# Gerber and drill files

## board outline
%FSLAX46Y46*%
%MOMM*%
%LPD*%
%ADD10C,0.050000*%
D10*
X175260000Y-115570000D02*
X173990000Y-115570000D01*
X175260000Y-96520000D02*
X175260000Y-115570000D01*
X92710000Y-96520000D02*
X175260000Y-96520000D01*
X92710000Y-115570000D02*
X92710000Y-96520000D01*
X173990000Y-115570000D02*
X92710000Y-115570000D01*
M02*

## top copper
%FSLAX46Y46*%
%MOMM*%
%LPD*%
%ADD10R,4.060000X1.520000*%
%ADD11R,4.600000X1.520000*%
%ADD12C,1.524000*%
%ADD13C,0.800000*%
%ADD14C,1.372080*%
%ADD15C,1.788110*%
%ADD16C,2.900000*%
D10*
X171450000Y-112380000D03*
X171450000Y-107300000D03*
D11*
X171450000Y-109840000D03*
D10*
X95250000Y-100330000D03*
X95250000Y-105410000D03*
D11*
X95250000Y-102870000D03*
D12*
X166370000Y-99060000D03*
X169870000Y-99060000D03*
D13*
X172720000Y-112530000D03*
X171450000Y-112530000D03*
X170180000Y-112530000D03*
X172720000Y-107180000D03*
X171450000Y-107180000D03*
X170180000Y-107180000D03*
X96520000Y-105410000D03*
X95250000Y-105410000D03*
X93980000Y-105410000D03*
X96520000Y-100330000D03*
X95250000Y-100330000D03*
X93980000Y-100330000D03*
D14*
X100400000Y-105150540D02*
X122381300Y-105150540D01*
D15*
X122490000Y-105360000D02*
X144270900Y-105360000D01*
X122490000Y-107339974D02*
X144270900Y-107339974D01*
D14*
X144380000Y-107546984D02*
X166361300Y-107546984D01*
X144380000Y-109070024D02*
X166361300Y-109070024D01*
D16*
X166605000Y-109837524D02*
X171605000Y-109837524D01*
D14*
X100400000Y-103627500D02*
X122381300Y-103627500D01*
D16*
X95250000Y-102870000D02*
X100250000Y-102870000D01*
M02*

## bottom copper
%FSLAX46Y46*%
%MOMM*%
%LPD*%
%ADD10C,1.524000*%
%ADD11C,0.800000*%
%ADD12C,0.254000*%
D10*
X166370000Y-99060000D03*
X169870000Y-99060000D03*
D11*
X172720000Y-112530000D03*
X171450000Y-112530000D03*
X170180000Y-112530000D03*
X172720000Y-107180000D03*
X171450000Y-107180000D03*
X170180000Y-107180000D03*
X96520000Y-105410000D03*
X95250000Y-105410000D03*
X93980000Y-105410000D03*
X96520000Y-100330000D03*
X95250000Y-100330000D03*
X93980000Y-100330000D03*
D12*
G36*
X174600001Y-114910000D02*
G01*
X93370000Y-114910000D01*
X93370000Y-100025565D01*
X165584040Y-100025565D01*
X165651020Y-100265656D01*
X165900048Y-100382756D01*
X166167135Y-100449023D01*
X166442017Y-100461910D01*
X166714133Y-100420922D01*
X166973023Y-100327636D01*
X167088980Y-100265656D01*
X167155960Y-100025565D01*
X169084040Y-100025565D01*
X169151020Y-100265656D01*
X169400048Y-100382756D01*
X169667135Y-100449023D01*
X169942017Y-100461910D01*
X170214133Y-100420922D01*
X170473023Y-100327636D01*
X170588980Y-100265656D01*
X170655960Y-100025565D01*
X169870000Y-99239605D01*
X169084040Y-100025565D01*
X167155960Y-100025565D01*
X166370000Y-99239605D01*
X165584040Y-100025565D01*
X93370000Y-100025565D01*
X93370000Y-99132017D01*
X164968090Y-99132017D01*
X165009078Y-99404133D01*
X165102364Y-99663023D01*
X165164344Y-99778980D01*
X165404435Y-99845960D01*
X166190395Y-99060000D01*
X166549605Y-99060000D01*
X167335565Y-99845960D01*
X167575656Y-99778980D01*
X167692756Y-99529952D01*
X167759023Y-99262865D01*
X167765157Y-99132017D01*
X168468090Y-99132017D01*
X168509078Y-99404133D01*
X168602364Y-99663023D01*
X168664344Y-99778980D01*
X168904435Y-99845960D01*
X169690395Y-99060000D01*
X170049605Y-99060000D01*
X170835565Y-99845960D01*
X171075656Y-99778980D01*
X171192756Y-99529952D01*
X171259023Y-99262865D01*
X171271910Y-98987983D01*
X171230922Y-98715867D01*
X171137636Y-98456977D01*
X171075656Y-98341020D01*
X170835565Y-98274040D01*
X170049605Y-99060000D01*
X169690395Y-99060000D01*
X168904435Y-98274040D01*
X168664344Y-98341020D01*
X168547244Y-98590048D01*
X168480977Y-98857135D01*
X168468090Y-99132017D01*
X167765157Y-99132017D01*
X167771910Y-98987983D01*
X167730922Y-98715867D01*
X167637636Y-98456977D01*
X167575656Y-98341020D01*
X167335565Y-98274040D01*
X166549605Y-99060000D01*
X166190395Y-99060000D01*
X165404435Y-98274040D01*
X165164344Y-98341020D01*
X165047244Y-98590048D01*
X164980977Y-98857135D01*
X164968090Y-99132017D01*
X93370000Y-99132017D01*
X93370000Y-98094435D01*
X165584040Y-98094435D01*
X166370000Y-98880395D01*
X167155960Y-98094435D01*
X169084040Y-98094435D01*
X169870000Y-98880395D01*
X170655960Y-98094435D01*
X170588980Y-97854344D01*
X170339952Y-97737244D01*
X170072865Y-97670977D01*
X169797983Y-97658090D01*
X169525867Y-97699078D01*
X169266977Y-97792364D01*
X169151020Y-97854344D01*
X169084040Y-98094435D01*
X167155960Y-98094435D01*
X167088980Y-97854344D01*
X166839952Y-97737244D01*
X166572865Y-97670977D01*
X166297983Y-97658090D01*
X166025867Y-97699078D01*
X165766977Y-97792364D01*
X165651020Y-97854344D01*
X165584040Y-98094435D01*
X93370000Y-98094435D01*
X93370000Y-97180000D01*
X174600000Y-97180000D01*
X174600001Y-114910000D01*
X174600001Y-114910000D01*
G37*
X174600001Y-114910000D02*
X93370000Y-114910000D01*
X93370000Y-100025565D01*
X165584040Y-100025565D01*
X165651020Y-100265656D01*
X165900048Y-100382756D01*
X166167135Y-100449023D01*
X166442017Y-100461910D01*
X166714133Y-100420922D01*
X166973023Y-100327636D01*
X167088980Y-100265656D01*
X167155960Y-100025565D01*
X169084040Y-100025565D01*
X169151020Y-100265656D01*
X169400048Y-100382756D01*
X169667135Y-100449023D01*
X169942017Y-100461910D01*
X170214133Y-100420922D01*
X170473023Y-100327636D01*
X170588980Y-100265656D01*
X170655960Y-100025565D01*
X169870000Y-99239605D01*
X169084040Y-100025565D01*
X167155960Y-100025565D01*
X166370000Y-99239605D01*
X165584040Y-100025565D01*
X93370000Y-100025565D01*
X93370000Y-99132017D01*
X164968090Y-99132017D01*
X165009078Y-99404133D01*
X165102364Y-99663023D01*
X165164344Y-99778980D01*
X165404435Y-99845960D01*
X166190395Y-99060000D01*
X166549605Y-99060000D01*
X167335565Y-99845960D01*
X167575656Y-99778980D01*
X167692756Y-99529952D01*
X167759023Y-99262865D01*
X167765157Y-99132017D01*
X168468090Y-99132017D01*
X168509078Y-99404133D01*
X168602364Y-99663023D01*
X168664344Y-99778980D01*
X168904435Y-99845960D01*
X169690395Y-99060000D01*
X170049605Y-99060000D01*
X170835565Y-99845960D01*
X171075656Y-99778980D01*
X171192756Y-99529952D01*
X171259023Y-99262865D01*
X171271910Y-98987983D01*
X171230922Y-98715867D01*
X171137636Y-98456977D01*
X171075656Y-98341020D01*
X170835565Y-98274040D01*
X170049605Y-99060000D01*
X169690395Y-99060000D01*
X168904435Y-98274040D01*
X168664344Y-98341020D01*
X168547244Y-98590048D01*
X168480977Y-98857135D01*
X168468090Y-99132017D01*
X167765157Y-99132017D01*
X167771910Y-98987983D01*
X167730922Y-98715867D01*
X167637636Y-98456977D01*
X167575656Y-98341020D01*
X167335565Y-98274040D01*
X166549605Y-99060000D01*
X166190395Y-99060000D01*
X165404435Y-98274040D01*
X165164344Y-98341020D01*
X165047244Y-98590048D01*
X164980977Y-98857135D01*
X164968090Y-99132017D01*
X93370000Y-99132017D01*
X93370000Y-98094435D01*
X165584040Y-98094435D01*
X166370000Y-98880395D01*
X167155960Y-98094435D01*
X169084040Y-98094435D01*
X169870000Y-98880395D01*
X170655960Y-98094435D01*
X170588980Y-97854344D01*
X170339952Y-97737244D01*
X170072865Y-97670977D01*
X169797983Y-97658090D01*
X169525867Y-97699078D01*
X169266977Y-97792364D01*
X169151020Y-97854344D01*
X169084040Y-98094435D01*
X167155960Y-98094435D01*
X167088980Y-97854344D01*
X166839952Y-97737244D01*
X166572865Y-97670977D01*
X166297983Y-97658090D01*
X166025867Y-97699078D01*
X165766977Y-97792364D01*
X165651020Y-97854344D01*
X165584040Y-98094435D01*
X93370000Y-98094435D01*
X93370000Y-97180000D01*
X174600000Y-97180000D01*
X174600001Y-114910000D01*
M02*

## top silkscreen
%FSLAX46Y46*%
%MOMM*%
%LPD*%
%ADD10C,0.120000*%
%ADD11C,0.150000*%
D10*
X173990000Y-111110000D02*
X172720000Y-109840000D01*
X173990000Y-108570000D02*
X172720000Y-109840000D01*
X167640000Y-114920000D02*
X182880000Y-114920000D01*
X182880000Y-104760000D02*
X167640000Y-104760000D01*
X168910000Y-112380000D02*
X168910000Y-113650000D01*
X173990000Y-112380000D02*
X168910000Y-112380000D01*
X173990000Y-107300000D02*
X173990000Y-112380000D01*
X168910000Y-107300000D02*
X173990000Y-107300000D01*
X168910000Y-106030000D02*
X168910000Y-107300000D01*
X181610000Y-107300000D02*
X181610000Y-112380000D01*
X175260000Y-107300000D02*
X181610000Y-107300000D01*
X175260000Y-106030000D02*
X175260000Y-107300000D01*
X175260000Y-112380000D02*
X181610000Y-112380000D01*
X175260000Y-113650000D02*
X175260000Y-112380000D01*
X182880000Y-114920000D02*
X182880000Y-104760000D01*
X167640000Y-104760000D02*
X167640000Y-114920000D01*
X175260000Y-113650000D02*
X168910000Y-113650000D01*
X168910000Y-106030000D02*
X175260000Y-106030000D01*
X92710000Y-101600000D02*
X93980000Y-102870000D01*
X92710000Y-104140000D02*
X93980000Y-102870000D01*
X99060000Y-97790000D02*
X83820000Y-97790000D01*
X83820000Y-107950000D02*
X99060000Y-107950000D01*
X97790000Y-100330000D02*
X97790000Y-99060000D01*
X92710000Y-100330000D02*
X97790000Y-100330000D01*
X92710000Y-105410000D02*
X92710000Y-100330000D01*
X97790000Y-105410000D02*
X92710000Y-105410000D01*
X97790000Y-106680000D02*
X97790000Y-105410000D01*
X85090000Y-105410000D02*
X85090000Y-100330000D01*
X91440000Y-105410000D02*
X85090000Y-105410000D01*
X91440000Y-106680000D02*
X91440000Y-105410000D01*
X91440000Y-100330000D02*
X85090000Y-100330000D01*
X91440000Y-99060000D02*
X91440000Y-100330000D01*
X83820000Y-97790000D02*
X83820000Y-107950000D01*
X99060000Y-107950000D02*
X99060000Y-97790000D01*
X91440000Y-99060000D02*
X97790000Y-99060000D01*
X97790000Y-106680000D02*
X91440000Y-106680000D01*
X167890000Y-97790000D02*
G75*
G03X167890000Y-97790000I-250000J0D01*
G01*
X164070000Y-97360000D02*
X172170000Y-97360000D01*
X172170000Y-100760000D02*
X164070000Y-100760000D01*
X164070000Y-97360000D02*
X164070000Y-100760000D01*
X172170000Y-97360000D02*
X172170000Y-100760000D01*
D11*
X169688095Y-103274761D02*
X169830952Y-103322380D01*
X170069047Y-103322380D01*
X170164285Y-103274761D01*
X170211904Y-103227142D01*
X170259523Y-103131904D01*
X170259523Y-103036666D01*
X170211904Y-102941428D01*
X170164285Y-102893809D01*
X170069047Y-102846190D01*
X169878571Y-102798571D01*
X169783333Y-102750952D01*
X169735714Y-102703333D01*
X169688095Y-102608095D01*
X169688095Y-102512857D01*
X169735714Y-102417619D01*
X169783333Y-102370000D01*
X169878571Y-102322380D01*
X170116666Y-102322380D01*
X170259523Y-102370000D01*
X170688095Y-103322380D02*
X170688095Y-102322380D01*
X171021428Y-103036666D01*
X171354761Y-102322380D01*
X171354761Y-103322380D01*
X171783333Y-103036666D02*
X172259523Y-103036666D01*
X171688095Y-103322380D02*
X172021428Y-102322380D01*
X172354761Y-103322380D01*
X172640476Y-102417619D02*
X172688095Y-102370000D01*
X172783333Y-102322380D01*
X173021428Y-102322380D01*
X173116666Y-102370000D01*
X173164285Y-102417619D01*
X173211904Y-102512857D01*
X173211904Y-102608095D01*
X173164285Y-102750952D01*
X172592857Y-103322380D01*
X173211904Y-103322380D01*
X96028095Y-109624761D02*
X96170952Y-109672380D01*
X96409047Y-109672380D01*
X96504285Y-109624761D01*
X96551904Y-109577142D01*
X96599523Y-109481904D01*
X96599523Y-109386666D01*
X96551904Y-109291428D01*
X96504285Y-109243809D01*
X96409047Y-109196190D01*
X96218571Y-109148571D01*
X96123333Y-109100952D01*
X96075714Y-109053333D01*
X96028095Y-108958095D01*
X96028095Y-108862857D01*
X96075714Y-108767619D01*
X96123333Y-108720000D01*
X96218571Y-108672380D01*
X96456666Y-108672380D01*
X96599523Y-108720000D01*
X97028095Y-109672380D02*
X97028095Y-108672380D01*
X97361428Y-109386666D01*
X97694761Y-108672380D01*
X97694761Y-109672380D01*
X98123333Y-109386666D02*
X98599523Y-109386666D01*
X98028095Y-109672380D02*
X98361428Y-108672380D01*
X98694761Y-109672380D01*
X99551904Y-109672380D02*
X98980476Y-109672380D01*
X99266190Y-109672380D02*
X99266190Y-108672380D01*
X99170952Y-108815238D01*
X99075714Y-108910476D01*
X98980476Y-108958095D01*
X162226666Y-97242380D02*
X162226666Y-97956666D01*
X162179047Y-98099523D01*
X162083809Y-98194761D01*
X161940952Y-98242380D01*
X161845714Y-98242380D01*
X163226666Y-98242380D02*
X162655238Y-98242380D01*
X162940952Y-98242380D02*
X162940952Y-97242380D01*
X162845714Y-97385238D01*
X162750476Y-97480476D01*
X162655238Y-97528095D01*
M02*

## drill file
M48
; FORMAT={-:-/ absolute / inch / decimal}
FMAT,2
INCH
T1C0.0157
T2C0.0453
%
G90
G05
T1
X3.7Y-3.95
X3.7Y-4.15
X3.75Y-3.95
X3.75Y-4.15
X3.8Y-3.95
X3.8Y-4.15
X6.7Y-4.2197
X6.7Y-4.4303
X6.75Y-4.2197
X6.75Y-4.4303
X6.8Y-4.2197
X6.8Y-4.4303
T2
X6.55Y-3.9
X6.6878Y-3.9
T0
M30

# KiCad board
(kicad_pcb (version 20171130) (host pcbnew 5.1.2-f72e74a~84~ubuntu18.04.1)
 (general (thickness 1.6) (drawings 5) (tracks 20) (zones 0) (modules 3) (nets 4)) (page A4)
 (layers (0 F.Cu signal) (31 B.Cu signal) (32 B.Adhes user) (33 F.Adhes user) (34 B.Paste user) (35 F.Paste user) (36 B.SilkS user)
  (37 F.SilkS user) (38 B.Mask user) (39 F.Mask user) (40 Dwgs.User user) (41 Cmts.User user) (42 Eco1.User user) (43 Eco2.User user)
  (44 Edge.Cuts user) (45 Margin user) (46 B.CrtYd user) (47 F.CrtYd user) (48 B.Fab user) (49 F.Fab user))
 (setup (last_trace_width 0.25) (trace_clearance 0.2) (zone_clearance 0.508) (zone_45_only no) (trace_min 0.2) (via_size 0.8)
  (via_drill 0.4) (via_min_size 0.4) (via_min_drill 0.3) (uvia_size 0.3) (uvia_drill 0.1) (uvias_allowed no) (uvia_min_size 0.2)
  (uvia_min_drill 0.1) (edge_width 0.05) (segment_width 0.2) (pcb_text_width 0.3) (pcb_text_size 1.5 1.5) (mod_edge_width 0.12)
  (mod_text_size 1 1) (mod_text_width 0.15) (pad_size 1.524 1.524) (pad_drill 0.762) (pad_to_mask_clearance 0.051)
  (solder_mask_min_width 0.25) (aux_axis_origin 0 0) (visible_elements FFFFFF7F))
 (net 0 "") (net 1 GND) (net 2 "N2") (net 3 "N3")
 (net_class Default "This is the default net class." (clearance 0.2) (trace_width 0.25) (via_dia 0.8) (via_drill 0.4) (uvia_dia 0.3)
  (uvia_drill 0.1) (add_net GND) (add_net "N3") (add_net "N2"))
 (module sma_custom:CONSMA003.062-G (layer F.Cu) (at 175.26 112.38)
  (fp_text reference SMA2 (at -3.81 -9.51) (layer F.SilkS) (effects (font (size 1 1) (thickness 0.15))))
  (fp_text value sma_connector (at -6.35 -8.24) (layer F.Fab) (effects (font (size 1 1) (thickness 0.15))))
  (fp_line (start -1.27 -1.27) (end -2.54 -2.54) (layer F.SilkS) (width 0.12))
  (fp_line (start -1.27 -3.81) (end -2.54 -2.54) (layer F.SilkS) (width 0.12))
  (fp_line (start -7.62 2.54) (end 7.62 2.54) (layer F.SilkS) (width 0.12))
  (fp_line (start 7.62 -7.62) (end -7.62 -7.62) (layer F.SilkS) (width 0.12))
  (fp_line (start -6.35 0) (end -6.35 1.27) (layer F.SilkS) (width 0.12))
  (fp_line (start -1.27 0) (end -6.35 0) (layer F.SilkS) (width 0.12))
  (fp_line (start -1.27 -5.08) (end -1.27 0) (layer F.SilkS) (width 0.12))
  (fp_line (start -6.35 -5.08) (end -1.27 -5.08) (layer F.SilkS) (width 0.12))
  (fp_line (start -6.35 -6.35) (end -6.35 -5.08) (layer F.SilkS) (width 0.12))
  (fp_line (start 6.35 -5.08) (end 6.35 0) (layer F.SilkS) (width 0.12))
  (fp_line (start 0 -5.08) (end 6.35 -5.08) (layer F.SilkS) (width 0.12))
  (fp_line (start 0 -6.35) (end 0 -5.08) (layer F.SilkS) (width 0.12))
  (fp_line (start 0 0) (end 6.35 0) (layer F.SilkS) (width 0.12))
  (fp_line (start 0 1.27) (end 0 0) (layer F.SilkS) (width 0.12))
  (fp_line (start 7.62 2.54) (end 7.62 -7.62) (layer F.SilkS) (width 0.12))
  (fp_line (start -7.62 -7.62) (end -7.62 2.54) (layer F.SilkS) (width 0.12))
  (fp_line (start 0 1.27) (end -6.35 1.27) (layer F.SilkS) (width 0.12))
  (fp_line (start -6.35 -6.35) (end 0 -6.35) (layer F.SilkS) (width 0.12))
  (pad 3 smd rect (at -3.81 0) (size 4.06 1.52) (layers F.Cu F.Paste F.Mask) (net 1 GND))
  (pad 2 smd rect (at -3.81 -5.08) (size 4.06 1.52) (layers F.Cu F.Paste F.Mask) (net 1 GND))
  (pad 1 smd rect (at -3.81 -2.54) (size 4.6 1.52) (layers F.Cu F.Paste F.Mask) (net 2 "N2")))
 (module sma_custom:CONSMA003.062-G (layer F.Cu) (at 91.44 100.33 180)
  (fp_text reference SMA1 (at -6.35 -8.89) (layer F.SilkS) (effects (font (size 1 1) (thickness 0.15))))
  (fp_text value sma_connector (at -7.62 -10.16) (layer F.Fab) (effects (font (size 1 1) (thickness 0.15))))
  (fp_line (start -1.27 -1.27) (end -2.54 -2.54) (layer F.SilkS) (width 0.12))
  (fp_line (start -1.27 -3.81) (end -2.54 -2.54) (layer F.SilkS) (width 0.12))
  (fp_line (start -7.62 2.54) (end 7.62 2.54) (layer F.SilkS) (width 0.12))
  (fp_line (start 7.62 -7.62) (end -7.62 -7.62) (layer F.SilkS) (width 0.12))
  (fp_line (start -6.35 0) (end -6.35 1.27) (layer F.SilkS) (width 0.12))
  (fp_line (start -1.27 0) (end -6.35 0) (layer F.SilkS) (width 0.12))
  (fp_line (start -1.27 -5.08) (end -1.27 0) (layer F.SilkS) (width 0.12))
  (fp_line (start -6.35 -5.08) (end -1.27 -5.08) (layer F.SilkS) (width 0.12))
  (fp_line (start -6.35 -6.35) (end -6.35 -5.08) (layer F.SilkS) (width 0.12))
  (fp_line (start 6.35 -5.08) (end 6.35 0) (layer F.SilkS) (width 0.12))
  (fp_line (start 0 -5.08) (end 6.35 -5.08) (layer F.SilkS) (width 0.12))
  (fp_line (start 0 -6.35) (end 0 -5.08) (layer F.SilkS) (width 0.12))
  (fp_line (start 0 0) (end 6.35 0) (layer F.SilkS) (width 0.12))
  (fp_line (start 0 1.27) (end 0 0) (layer F.SilkS) (width 0.12))
  (fp_line (start 7.62 2.54) (end 7.62 -7.62) (layer F.SilkS) (width 0.12))
  (fp_line (start -7.62 -7.62) (end -7.62 2.54) (layer F.SilkS) (width 0.12))
  (fp_line (start 0 1.27) (end -6.35 1.27) (layer F.SilkS) (width 0.12))
  (fp_line (start -6.35 -6.35) (end 0 -6.35) (layer F.SilkS) (width 0.12))
  (pad 3 smd rect (at -3.81 0 180) (size 4.06 1.52) (layers F.Cu F.Paste F.Mask) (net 1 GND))
  (pad 2 smd rect (at -3.81 -5.08 180) (size 4.06 1.52) (layers F.Cu F.Paste F.Mask) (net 1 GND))
  (pad 1 smd rect (at -3.81 -2.54 180) (size 4.6 1.52) (layers F.Cu F.Paste F.Mask) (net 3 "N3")))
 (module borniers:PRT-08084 (layer F.Cu) (at 166.37 93.98 180)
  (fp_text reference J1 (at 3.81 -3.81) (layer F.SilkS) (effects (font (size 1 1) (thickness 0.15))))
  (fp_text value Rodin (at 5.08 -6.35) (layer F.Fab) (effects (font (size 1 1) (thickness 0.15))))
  (fp_circle (center -1.27 -3.81) (end -1.02 -3.81) (layer F.SilkS) (width 0.12))
  (fp_line (start 2.3 -3.38) (end -5.8 -3.38) (layer F.SilkS) (width 0.12))
  (fp_line (start -5.8 -6.78) (end 2.3 -6.78) (layer F.SilkS) (width 0.12))
  (fp_line (start 2.3 -3.38) (end 2.3 -6.78) (layer F.SilkS) (width 0.12))
  (fp_line (start -5.8 -3.38) (end -5.8 -6.78) (layer F.SilkS) (width 0.12))
  (pad 2 thru_hole circle (at 0 -5.08 180) (size 1.524 1.524) (drill 1.15) (layers *.Cu *.Mask) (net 1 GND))
  (pad 1 thru_hole circle (at -3.5 -5.08 180) (size 1.524 1.524) (drill 1.15) (layers *.Cu *.Mask) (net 1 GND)))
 (gr_line (start 175.26 115.57) (end 173.99 115.57) (layer Edge.Cuts) (width 0.05))
 (gr_line (start 175.26 96.52) (end 175.26 115.57) (layer Edge.Cuts) (width 0.05))
 (gr_line (start 92.71 96.52) (end 175.26 96.52) (layer Edge.Cuts) (width 0.05))
 (gr_line (start 92.71 115.57) (end 92.71 96.52) (layer Edge.Cuts) (width 0.05))
 (gr_line (start 173.99 115.57) (end 92.71 115.57) (layer Edge.Cuts) (width 0.05))
 (segment (start 100.4 105.15054) (end 122.3813 105.15054) (width 1.37208) (layer F.Cu) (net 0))
 (segment (start 122.49 105.36) (end 144.2709 105.36) (width 1.78811) (layer F.Cu) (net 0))
 (segment (start 122.49 107.339974) (end 144.2709 107.339974) (width 1.78811) (layer F.Cu) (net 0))
 (segment (start 144.38 107.546984) (end 166.3613 107.546984) (width 1.37208) (layer F.Cu) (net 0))
 (via (at 172.72 112.53) (size 0.8) (drill 0.4) (layers F.Cu B.Cu) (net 1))
 (via (at 171.45 112.53) (size 0.8) (drill 0.4) (layers F.Cu B.Cu) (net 1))
 (via (at 170.18 112.53) (size 0.8) (drill 0.4) (layers F.Cu B.Cu) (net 1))
 (via (at 172.72 107.18) (size 0.8) (drill 0.4) (layers F.Cu B.Cu) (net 1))
 (via (at 171.45 107.18) (size 0.8) (drill 0.4) (layers F.Cu B.Cu) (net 1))
 (via (at 170.18 107.18) (size 0.8) (drill 0.4) (layers F.Cu B.Cu) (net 1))
 (segment (start 144.38 109.070024) (end 166.3613 109.070024) (width 1.37208) (layer F.Cu) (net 2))
 (segment (start 166.605 109.837524) (end 171.605 109.837524) (width 2.9) (layer F.Cu) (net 2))
 (segment (start 100.4 103.6275) (end 122.3813 103.6275) (width 1.37208) (layer F.Cu) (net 3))
 (segment (start 95.25 102.87) (end 100.25 102.87) (width 2.9) (layer F.Cu) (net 3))
 (via (at 96.52 105.41) (size 0.8) (drill 0.4) (layers F.Cu B.Cu) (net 1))
 (via (at 95.25 105.41) (size 0.8) (drill 0.4) (layers F.Cu B.Cu) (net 1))
 (via (at 93.98 105.41) (size 0.8) (drill 0.4) (layers F.Cu B.Cu) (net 1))
 (via (at 96.52 100.33) (size 0.8) (drill 0.4) (layers F.Cu B.Cu) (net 1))
 (via (at 95.25 100.33) (size 0.8) (drill 0.4) (layers F.Cu B.Cu) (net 1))
 (via (at 93.98 100.33) (size 0.8) (drill 0.4) (layers F.Cu B.Cu) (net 1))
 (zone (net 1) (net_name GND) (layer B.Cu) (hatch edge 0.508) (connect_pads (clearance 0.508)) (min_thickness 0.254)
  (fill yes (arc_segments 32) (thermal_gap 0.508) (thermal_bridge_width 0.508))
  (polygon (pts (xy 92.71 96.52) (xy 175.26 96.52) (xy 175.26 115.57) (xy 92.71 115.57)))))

